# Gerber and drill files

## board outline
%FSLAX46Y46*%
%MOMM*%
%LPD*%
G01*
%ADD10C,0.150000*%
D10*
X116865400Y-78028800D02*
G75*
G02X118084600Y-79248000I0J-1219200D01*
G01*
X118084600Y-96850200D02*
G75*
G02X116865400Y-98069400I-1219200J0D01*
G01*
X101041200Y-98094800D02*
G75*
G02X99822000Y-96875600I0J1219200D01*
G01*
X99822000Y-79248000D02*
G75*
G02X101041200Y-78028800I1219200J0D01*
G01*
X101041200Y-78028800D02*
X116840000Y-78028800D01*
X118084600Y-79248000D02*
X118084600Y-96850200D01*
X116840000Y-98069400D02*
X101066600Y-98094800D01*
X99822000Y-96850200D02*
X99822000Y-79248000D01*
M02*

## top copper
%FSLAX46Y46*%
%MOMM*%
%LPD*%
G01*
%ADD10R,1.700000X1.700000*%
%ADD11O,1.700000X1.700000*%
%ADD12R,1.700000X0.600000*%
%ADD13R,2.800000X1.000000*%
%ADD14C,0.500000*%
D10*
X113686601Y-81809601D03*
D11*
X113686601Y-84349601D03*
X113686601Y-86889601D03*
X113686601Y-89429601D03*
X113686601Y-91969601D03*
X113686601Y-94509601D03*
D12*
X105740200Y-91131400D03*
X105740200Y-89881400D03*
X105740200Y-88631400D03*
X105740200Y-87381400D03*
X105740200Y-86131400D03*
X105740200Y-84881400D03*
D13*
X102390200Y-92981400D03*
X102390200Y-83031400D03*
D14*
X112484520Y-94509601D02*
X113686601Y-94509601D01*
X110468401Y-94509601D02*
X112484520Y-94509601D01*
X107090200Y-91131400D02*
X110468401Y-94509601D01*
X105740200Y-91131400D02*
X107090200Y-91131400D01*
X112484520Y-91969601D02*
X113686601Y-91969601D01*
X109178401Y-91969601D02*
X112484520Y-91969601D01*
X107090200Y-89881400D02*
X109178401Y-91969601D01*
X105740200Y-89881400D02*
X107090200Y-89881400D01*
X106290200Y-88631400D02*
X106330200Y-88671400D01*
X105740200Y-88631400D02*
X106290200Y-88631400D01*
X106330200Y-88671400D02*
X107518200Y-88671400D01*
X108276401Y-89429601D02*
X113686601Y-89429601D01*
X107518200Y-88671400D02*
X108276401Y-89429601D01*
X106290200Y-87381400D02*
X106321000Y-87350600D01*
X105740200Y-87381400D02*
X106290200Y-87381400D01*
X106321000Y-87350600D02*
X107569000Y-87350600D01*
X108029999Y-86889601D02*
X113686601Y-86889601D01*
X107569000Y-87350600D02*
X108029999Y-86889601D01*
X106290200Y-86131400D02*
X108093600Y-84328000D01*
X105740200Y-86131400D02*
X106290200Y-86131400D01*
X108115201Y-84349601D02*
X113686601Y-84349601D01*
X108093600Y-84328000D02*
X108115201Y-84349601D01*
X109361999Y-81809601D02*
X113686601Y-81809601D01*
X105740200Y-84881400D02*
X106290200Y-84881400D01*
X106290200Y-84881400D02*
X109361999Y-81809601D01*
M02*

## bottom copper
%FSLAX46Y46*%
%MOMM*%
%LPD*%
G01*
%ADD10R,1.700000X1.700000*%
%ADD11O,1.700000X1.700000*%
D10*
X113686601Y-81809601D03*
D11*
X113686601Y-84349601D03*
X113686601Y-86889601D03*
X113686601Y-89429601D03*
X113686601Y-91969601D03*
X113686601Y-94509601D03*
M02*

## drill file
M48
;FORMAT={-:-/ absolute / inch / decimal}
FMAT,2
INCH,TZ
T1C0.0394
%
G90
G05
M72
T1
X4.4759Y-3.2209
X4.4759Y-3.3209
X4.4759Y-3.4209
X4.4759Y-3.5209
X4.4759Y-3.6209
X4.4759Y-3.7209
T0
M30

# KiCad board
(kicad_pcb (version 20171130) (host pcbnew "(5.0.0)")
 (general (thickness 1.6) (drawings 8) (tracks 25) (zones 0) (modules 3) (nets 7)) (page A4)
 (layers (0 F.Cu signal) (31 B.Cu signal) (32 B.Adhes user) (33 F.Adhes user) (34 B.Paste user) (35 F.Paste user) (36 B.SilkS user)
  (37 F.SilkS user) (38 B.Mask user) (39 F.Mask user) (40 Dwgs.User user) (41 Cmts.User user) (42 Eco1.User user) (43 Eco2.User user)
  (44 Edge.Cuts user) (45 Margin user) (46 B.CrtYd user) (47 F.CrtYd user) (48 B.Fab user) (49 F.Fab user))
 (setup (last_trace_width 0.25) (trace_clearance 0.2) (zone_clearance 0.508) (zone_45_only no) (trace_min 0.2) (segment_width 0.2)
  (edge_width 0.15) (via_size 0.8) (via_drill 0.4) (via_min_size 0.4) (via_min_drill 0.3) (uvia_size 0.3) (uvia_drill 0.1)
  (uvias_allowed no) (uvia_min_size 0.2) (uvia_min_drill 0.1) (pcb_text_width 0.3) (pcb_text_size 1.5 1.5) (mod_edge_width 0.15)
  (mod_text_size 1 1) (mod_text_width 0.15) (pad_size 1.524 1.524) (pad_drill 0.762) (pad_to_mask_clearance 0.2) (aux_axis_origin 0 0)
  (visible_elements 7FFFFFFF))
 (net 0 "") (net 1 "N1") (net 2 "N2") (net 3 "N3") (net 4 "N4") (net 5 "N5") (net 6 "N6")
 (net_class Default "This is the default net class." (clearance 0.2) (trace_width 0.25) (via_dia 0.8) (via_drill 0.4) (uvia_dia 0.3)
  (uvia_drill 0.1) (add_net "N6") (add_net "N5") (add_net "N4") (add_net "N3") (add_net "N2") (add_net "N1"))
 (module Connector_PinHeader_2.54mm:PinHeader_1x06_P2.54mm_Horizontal (layer F.Cu) (at 113.686601 81.809601)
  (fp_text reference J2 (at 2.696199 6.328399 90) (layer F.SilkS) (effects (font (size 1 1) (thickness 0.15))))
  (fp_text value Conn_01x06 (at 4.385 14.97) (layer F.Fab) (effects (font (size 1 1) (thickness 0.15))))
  (pad 1 thru_hole rect (at 0 0) (size 1.7 1.7) (drill 1) (layers *.Cu *.Mask) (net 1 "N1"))
  (pad 2 thru_hole oval (at 0 2.54) (size 1.7 1.7) (drill 1) (layers *.Cu *.Mask) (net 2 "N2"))
  (pad 3 thru_hole oval (at 0 5.08) (size 1.7 1.7) (drill 1) (layers *.Cu *.Mask) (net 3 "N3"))
  (pad 4 thru_hole oval (at 0 7.62) (size 1.7 1.7) (drill 1) (layers *.Cu *.Mask) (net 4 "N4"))
  (pad 5 thru_hole oval (at 0 10.16) (size 1.7 1.7) (drill 1) (layers *.Cu *.Mask) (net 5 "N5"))
  (pad 6 thru_hole oval (at 0 12.7) (size 1.7 1.7) (drill 1) (layers *.Cu *.Mask) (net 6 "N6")))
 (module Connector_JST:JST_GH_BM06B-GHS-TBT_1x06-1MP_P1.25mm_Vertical (layer F.Cu) (at 103.7902 88.0064 90)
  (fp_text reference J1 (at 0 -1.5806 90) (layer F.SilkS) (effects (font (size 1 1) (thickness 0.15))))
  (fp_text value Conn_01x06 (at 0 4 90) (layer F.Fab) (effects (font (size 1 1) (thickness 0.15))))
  (pad 1 smd rect (at -3.125 1.95 90) (size 0.6 1.7) (layers F.Cu F.Paste F.Mask) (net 6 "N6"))
  (pad 2 smd rect (at -1.875 1.95 90) (size 0.6 1.7) (layers F.Cu F.Paste F.Mask) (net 5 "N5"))
  (pad 3 smd rect (at -0.625 1.95 90) (size 0.6 1.7) (layers F.Cu F.Paste F.Mask) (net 4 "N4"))
  (pad 4 smd rect (at 0.625 1.95 90) (size 0.6 1.7) (layers F.Cu F.Paste F.Mask) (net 3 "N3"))
  (pad 5 smd rect (at 1.875 1.95 90) (size 0.6 1.7) (layers F.Cu F.Paste F.Mask) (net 2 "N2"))
  (pad 6 smd rect (at 3.125 1.95 90) (size 0.6 1.7) (layers F.Cu F.Paste F.Mask) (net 1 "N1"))
  (pad MP smd rect (at -4.975 -1.4 90) (size 1 2.8) (layers F.Cu F.Paste F.Mask))
  (pad MP smd rect (at 4.975 -1.4 90) (size 1 2.8) (layers F.Cu F.Paste F.Mask)))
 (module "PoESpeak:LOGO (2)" (layer F.Cu) (at 109.6264 88.0872 90)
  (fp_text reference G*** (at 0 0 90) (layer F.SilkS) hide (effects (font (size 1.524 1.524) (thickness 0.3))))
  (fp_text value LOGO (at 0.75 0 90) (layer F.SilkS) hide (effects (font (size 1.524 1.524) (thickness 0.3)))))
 (gr_arc (start 116.8654 79.248) (end 118.0846 79.248) (angle -90) (layer Edge.Cuts) (width 0.15))
 (gr_arc (start 116.8654 96.8502) (end 116.8654 98.0694) (angle -90) (layer Edge.Cuts) (width 0.15))
 (gr_arc (start 101.0412 96.8756) (end 99.822 96.8756) (angle -90) (layer Edge.Cuts) (width 0.15))
 (gr_arc (start 101.0412 79.248) (end 101.0412 78.0288) (angle -90) (layer Edge.Cuts) (width 0.15))
 (gr_line (start 101.0412 78.0288) (end 116.84 78.0288) (layer Edge.Cuts) (width 0.15))
 (gr_line (start 118.0846 79.248) (end 118.0846 96.8502) (layer Edge.Cuts) (width 0.15))
 (gr_line (start 116.84 98.0694) (end 101.0666 98.0948) (layer Edge.Cuts) (width 0.15))
 (gr_line (start 99.822 96.8502) (end 99.822 79.248) (layer Edge.Cuts) (width 0.15))
 (segment (start 112.48452 94.509601) (end 113.686601 94.509601) (width 0.5) (layer F.Cu) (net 6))
 (segment (start 110.468401 94.509601) (end 112.48452 94.509601) (width 0.5) (layer F.Cu) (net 6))
 (segment (start 107.0902 91.1314) (end 110.468401 94.509601) (width 0.5) (layer F.Cu) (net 6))
 (segment (start 105.7402 91.1314) (end 107.0902 91.1314) (width 0.5) (layer F.Cu) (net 6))
 (segment (start 112.48452 91.969601) (end 113.686601 91.969601) (width 0.5) (layer F.Cu) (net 5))
 (segment (start 109.178401 91.969601) (end 112.48452 91.969601) (width 0.5) (layer F.Cu) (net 5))
 (segment (start 107.0902 89.8814) (end 109.178401 91.969601) (width 0.5) (layer F.Cu) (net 5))
 (segment (start 105.7402 89.8814) (end 107.0902 89.8814) (width 0.5) (layer F.Cu) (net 5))
 (segment (start 106.2902 88.6314) (end 106.3302 88.6714) (width 0.5) (layer F.Cu) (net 4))
 (segment (start 105.7402 88.6314) (end 106.2902 88.6314) (width 0.5) (layer F.Cu) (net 4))
 (segment (start 106.3302 88.6714) (end 107.5182 88.6714) (width 0.5) (layer F.Cu) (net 4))
 (segment (start 108.276401 89.429601) (end 113.686601 89.429601) (width 0.5) (layer F.Cu) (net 4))
 (segment (start 107.5182 88.6714) (end 108.276401 89.429601) (width 0.5) (layer F.Cu) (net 4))
 (segment (start 106.2902 87.3814) (end 106.321 87.3506) (width 0.5) (layer F.Cu) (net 3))
 (segment (start 105.7402 87.3814) (end 106.2902 87.3814) (width 0.5) (layer F.Cu) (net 3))
 (segment (start 106.321 87.3506) (end 107.569 87.3506) (width 0.5) (layer F.Cu) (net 3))
 (segment (start 108.029999 86.889601) (end 113.686601 86.889601) (width 0.5) (layer F.Cu) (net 3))
 (segment (start 107.569 87.3506) (end 108.029999 86.889601) (width 0.5) (layer F.Cu) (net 3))
 (segment (start 106.2902 86.1314) (end 108.0936 84.328) (width 0.5) (layer F.Cu) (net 2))
 (segment (start 105.7402 86.1314) (end 106.2902 86.1314) (width 0.5) (layer F.Cu) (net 2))
 (segment (start 108.115201 84.349601) (end 113.686601 84.349601) (width 0.5) (layer F.Cu) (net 2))
 (segment (start 108.0936 84.328) (end 108.115201 84.349601) (width 0.5) (layer F.Cu) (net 2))
 (segment (start 109.361999 81.809601) (end 113.686601 81.809601) (width 0.5) (layer F.Cu) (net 1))
 (segment (start 105.7402 84.8814) (end 106.2902 84.8814) (width 0.5) (layer F.Cu) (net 1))
 (segment (start 106.2902 84.8814) (end 109.361999 81.809601) (width 0.5) (layer F.Cu) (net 1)))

